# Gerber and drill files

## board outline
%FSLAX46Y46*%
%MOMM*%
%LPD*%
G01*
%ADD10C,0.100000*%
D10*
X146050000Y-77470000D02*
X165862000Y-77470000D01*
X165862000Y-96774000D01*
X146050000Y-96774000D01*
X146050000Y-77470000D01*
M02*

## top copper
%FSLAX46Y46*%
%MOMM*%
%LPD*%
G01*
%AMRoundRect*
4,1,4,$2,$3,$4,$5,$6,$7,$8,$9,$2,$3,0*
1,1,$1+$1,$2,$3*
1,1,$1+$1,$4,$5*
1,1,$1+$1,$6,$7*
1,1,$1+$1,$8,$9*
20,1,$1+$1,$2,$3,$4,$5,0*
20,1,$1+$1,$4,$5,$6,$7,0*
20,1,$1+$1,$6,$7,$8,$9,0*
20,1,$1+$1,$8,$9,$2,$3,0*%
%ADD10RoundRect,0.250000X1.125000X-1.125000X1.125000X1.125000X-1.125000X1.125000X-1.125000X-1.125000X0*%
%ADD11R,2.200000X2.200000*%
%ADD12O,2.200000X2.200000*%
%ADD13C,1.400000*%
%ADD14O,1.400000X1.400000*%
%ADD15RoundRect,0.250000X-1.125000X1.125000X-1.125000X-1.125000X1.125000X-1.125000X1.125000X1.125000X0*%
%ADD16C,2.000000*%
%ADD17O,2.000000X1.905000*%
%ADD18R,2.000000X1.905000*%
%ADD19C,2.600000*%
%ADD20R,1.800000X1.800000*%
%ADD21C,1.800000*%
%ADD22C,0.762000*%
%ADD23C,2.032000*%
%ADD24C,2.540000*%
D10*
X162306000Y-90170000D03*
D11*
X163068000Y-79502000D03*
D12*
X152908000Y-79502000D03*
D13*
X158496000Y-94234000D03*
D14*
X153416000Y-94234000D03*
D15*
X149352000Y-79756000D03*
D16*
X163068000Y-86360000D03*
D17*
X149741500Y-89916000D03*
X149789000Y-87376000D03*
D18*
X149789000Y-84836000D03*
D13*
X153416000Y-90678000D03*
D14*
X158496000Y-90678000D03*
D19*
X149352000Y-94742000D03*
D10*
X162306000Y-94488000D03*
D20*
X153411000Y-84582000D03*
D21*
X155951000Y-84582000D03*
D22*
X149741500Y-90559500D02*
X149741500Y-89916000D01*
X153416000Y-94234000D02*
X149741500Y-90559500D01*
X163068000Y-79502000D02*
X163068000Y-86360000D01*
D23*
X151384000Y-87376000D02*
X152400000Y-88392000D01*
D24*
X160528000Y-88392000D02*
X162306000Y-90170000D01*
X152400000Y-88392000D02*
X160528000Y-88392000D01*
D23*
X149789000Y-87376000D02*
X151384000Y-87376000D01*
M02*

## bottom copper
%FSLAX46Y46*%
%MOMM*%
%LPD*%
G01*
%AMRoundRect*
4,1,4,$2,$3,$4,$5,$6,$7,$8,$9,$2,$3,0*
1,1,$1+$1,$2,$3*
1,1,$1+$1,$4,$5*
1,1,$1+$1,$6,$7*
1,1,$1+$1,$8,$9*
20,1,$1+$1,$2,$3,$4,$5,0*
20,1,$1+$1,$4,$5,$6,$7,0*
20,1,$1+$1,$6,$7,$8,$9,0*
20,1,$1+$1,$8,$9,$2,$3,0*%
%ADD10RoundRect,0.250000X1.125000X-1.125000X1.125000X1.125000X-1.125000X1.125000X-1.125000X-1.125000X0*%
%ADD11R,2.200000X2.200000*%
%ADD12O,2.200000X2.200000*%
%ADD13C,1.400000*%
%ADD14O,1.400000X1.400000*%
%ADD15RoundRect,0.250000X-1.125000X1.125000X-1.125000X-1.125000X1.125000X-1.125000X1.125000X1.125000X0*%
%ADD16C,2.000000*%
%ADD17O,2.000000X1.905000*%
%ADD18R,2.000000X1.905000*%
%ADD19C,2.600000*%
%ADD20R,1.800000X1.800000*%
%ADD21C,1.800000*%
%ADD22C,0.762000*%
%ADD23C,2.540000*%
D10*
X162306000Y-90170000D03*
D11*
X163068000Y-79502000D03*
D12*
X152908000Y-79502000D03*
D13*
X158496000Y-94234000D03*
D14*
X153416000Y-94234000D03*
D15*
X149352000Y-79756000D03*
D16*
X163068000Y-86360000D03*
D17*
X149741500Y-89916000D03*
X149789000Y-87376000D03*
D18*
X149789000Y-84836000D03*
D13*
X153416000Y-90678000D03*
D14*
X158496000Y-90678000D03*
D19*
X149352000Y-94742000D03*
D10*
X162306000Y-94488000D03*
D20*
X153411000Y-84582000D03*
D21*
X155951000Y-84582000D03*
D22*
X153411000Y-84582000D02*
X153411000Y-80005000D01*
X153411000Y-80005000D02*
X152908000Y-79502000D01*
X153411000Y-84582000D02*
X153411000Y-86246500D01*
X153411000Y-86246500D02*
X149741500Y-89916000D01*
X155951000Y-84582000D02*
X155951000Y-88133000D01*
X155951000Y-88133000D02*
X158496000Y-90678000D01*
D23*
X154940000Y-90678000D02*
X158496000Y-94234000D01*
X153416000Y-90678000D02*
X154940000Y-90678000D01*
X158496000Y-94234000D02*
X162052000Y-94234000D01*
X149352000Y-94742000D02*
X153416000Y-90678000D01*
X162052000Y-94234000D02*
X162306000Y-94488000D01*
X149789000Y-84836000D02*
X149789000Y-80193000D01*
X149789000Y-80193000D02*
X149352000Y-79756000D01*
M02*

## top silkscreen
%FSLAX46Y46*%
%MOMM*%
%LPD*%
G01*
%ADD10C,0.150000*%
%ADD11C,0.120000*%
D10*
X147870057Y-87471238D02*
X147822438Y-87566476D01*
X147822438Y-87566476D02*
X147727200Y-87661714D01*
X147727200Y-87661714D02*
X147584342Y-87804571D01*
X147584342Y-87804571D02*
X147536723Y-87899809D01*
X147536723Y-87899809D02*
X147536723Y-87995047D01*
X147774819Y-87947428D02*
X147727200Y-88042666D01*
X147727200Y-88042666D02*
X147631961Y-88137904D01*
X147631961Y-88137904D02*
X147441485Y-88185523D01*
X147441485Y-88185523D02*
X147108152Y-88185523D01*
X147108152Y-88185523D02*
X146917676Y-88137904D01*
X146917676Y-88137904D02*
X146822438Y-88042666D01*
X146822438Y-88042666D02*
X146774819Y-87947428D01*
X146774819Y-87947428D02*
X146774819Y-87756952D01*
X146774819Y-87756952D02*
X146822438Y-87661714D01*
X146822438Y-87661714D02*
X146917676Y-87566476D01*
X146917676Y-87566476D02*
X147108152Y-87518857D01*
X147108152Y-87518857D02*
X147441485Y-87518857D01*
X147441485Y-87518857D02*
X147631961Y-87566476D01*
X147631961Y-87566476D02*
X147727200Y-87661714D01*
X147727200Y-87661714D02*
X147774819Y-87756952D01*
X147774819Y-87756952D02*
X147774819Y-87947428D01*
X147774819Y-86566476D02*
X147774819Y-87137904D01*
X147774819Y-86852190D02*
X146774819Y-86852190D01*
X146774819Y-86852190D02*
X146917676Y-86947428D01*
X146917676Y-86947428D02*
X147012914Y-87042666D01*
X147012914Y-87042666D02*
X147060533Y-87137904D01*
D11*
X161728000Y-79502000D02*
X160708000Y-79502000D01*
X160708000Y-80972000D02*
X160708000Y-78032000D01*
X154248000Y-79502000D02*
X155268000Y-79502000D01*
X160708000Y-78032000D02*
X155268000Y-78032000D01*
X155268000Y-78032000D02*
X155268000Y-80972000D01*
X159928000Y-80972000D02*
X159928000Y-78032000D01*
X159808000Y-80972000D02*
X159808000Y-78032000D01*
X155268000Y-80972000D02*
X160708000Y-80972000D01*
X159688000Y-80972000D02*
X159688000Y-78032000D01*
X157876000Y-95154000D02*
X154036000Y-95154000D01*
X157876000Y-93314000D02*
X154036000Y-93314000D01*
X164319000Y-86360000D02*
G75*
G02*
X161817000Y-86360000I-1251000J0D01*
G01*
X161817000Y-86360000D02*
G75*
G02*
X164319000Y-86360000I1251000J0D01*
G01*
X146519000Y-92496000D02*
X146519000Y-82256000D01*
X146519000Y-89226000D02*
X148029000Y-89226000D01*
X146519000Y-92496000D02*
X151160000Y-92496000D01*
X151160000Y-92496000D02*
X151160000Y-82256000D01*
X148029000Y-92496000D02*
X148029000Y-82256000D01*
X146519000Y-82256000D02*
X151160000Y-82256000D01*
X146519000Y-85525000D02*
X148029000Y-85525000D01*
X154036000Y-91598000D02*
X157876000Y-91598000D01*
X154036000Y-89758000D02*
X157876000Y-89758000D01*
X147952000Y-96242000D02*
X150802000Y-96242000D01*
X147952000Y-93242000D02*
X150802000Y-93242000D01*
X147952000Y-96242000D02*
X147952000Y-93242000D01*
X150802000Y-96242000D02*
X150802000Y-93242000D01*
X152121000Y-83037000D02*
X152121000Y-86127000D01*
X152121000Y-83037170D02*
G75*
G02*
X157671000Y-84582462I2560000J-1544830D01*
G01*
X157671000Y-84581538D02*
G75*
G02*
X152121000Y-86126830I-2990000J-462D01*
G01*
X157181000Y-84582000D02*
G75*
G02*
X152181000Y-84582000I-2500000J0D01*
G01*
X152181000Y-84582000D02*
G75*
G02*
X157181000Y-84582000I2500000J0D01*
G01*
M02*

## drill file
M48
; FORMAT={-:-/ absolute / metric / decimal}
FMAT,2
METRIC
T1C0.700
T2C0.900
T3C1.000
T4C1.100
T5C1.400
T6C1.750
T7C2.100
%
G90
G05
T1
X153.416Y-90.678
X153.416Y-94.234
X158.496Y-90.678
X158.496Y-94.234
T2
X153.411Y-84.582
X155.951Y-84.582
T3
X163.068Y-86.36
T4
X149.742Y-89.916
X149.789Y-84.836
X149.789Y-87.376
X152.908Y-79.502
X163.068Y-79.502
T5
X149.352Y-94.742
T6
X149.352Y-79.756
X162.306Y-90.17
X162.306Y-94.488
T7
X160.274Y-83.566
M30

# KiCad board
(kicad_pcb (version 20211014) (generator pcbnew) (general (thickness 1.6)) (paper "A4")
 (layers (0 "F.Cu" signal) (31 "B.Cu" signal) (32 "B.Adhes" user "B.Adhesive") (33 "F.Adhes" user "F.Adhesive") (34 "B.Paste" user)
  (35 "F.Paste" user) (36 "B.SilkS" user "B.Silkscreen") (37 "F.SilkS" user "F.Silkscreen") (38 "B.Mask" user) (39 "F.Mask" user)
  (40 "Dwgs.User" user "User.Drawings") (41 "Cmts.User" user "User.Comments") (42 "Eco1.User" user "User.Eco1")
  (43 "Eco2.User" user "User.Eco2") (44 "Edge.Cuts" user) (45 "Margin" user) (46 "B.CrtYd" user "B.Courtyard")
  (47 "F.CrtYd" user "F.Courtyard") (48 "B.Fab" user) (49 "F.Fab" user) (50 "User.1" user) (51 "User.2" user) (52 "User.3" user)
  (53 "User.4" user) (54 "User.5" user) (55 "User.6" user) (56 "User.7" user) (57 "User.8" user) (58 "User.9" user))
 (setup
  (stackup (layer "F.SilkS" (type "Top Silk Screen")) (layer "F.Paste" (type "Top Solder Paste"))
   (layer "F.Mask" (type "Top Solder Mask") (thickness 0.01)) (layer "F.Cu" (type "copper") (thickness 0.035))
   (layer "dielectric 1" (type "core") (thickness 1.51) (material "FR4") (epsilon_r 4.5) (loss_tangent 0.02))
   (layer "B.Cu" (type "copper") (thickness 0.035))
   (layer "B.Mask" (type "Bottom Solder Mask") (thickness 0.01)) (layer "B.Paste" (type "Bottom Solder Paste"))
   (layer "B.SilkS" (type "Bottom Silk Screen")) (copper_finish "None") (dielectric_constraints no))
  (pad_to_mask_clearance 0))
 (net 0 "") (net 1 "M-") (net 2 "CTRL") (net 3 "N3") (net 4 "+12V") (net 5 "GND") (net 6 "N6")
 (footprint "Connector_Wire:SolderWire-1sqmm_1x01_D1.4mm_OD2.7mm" (layer "F.Cu") (at 162.306 90.17 90)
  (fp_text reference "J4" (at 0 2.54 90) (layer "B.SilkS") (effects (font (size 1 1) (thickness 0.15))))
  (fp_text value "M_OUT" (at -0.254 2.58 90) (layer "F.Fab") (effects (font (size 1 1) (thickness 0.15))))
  (pad "1" thru_hole roundrect (at 0 0 90) (size 2.75 2.75) (drill 1.75) (layers *.Cu *.Mask) (roundrect_rratio 0.090909) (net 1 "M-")))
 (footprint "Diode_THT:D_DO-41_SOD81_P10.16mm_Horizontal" (layer "F.Cu") (at 163.068 79.502 180)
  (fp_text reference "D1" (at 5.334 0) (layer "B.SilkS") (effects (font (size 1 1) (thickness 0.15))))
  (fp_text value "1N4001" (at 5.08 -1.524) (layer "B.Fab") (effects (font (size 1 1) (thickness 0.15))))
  (fp_line (start 1.34 0) (end 2.36 0) (layer "F.SilkS") (width 0.12))
  (fp_line (start 2.36 -1.47) (end 2.36 1.47) (layer "F.SilkS") (width 0.12))
  (fp_line (start 8.82 0) (end 7.8 0) (layer "F.SilkS") (width 0.12))
  (fp_line (start 2.36 1.47) (end 7.8 1.47) (layer "F.SilkS") (width 0.12))
  (fp_line (start 7.8 1.47) (end 7.8 -1.47) (layer "F.SilkS") (width 0.12))
  (fp_line (start 3.14 -1.47) (end 3.14 1.47) (layer "F.SilkS") (width 0.12))
  (fp_line (start 3.26 -1.47) (end 3.26 1.47) (layer "F.SilkS") (width 0.12))
  (fp_line (start 7.8 -1.47) (end 2.36 -1.47) (layer "F.SilkS") (width 0.12))
  (fp_line (start 3.38 -1.47) (end 3.38 1.47) (layer "F.SilkS") (width 0.12))
  (pad "1" thru_hole rect (at 0 0 180) (size 2.2 2.2) (drill 1.1) (layers *.Cu *.Mask) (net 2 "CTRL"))
  (pad "2" thru_hole oval (at 10.16 0 180) (size 2.2 2.2) (drill 1.1) (layers *.Cu *.Mask) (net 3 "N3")))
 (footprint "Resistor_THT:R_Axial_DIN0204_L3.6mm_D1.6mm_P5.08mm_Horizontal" (layer "F.Cu") (at 158.496 94.234 180)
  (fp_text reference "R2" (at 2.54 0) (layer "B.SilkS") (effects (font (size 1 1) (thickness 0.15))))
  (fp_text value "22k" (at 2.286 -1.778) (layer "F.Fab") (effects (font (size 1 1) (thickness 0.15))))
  (fp_line (start 0.62 -0.92) (end 4.46 -0.92) (layer "F.SilkS") (width 0.12))
  (fp_line (start 0.62 0.92) (end 4.46 0.92) (layer "F.SilkS") (width 0.12))
  (pad "1" thru_hole circle (at 0 0 180) (size 1.4 1.4) (drill 0.7) (layers *.Cu *.Mask) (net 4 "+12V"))
  (pad "2" thru_hole oval (at 5.08 0 180) (size 1.4 1.4) (drill 0.7) (layers *.Cu *.Mask) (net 3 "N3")))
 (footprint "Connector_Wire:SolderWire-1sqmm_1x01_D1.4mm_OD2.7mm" (layer "F.Cu") (at 149.352 79.756 -90)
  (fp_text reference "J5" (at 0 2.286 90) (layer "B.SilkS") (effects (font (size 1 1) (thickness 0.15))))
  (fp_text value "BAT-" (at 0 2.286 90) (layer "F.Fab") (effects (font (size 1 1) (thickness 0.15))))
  (pad "1" thru_hole roundrect (at 0 0 270) (size 2.75 2.75) (drill 1.75) (layers *.Cu *.Mask) (roundrect_rratio 0.090909) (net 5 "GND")))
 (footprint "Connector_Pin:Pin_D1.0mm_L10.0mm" (layer "F.Cu") (at 163.068 86.36 -90)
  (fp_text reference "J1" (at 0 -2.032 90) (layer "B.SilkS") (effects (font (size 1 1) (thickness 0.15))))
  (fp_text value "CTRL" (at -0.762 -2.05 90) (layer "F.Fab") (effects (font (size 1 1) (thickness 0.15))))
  (fp_circle (center 0 0) (end 1.25 0.05) (layer "F.SilkS") (width 0.12) (fill none))
  (pad "1" thru_hole circle (at 0 0 270) (size 2 2) (drill 1) (layers *.Cu *.Mask) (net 2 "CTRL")))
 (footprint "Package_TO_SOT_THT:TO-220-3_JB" (layer "F.Cu") (at 149.789 89.916 90)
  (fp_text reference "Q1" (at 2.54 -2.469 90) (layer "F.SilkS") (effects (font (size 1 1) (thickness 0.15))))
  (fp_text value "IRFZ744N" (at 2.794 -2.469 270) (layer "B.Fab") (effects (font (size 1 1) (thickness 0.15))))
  (fp_line (start -2.58 -3.27) (end 7.66 -3.27) (layer "F.SilkS") (width 0.12))
  (fp_line (start 0.69 -3.27) (end 0.69 -1.76) (layer "F.SilkS") (width 0.12))
  (fp_line (start -2.58 -3.27) (end -2.58 1.371) (layer "F.SilkS") (width 0.12))
  (fp_line (start -2.58 1.371) (end 7.66 1.371) (layer "F.SilkS") (width 0.12))
  (fp_line (start -2.58 -1.76) (end 7.66 -1.76) (layer "F.SilkS") (width 0.12))
  (fp_line (start 7.66 -3.27) (end 7.66 1.371) (layer "F.SilkS") (width 0.12))
  (fp_line (start 4.391 -3.27) (end 4.391 -1.76) (layer "F.SilkS") (width 0.12))
  (pad "1" thru_hole oval (at 0 -0.0475 90) (size 1.905 2) (drill 1.1) (layers *.Cu *.Mask) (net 3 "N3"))
  (pad "2" thru_hole oval (at 2.54 0 90) (size 1.905 2) (drill 1.1) (layers *.Cu *.Mask) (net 1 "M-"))
  (pad "3" thru_hole rect (at 5.08 0 90) (size 1.905 2) (drill 1.1) (layers *.Cu *.Mask) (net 5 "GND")))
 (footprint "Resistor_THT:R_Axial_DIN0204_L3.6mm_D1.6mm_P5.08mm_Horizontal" (layer "F.Cu") (at 153.416 90.678)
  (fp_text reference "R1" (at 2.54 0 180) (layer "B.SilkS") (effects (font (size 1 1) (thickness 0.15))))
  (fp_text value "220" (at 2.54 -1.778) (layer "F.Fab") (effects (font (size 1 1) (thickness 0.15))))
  (fp_line (start 0.62 0.92) (end 4.46 0.92) (layer "F.SilkS") (width 0.12))
  (fp_line (start 0.62 -0.92) (end 4.46 -0.92) (layer "F.SilkS") (width 0.12))
  (pad "1" thru_hole circle (at 0 0) (size 1.4 1.4) (drill 0.7) (layers *.Cu *.Mask) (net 4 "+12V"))
  (pad "2" thru_hole oval (at 5.08 0) (size 1.4 1.4) (drill 0.7) (layers *.Cu *.Mask) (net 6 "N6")))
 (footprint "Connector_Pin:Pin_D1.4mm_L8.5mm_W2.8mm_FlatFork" (layer "F.Cu") (at 149.352 94.742 90)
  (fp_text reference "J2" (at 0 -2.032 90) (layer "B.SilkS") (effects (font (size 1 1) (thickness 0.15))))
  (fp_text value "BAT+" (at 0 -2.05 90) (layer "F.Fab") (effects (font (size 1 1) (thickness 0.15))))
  (fp_line (start -1.5 -1.4) (end -1.5 1.45) (layer "F.SilkS") (width 0.12))
  (fp_line (start 1.5 -1.4) (end 1.5 1.45) (layer "F.SilkS") (width 0.12))
  (fp_line (start -1.5 -1.4) (end 1.5 -1.4) (layer "F.SilkS") (width 0.12))
  (fp_line (start -1.5 1.45) (end 1.5 1.45) (layer "F.SilkS") (width 0.12))
  (pad "1" thru_hole circle (at 0 0 90) (size 2.6 2.6) (drill 1.4) (layers *.Cu *.Mask) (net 4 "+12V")))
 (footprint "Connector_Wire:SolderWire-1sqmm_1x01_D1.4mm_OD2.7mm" (layer "F.Cu") (at 162.306 94.488 90)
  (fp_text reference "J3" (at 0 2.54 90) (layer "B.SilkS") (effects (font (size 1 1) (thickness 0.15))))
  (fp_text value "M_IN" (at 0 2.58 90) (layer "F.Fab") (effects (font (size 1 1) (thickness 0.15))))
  (pad "1" thru_hole roundrect (at 0 0 90) (size 2.75 2.75) (drill 1.75) (layers *.Cu *.Mask) (roundrect_rratio 0.090909) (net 4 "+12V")))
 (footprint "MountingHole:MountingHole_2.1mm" (layer "F.Cu") (at 160.274 83.566 90)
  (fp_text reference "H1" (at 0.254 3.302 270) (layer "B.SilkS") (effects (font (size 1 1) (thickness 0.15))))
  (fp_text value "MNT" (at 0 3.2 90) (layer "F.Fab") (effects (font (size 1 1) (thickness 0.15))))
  (pad "" np_thru_hole circle (at 0 0 90) (size 2.1 2.1) (drill 2.1) (layers *.Cu *.Mask)))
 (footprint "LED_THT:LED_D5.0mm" (layer "F.Cu") (at 153.411 84.582)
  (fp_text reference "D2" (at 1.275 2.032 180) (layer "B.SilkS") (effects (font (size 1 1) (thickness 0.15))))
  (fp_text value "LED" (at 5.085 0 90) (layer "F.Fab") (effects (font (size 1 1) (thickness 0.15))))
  (fp_line (start -1.29 -1.545) (end -1.29 1.545) (layer "F.SilkS") (width 0.12))
  (fp_arc (start -1.29 -1.54483) (mid 2.072002 -2.880433) (end 4.26 0.000462) (layer "F.SilkS") (width 0.12))
  (fp_arc (start 4.26 -0.000462) (mid 2.072002 2.880433) (end -1.29 1.54483) (layer "F.SilkS") (width 0.12))
  (fp_circle (center 1.27 0) (end 3.77 0) (layer "F.SilkS") (width 0.12) (fill none))
  (pad "1" thru_hole rect (at 0 0) (size 1.8 1.8) (drill 0.9) (layers *.Cu *.Mask) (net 3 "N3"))
  (pad "2" thru_hole circle (at 2.54 0) (size 1.8 1.8) (drill 0.9) (layers *.Cu *.Mask) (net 6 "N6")))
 (gr_rect (start 146.05 77.47) (end 165.862 96.774) (layer "Edge.Cuts") (width 0.1) (fill none))
 (segment (start 149.7415 90.5595) (end 149.7415 89.916) (width 0.762) (layer "F.Cu") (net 3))
 (segment (start 153.416 94.234) (end 149.7415 90.5595) (width 0.762) (layer "F.Cu") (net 3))
 (segment (start 153.411 84.582) (end 153.411 80.005) (width 0.762) (layer "B.Cu") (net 3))
 (segment (start 153.411 80.005) (end 152.908 79.502) (width 0.762) (layer "B.Cu") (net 3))
 (segment (start 153.411 84.582) (end 153.411 86.2465) (width 0.762) (layer "B.Cu") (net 3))
 (segment (start 153.411 86.2465) (end 149.7415 89.916) (width 0.762) (layer "B.Cu") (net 3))
 (segment (start 155.951 84.582) (end 155.951 88.133) (width 0.762) (layer "B.Cu") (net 6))
 (segment (start 155.951 88.133) (end 158.496 90.678) (width 0.762) (layer "B.Cu") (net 6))
 (segment (start 154.94 90.678) (end 158.496 94.234) (width 2.54) (layer "B.Cu") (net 4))
 (segment (start 153.416 90.678) (end 154.94 90.678) (width 2.54) (layer "B.Cu") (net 4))
 (segment (start 158.496 94.234) (end 162.052 94.234) (width 2.54) (layer "B.Cu") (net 4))
 (segment (start 149.352 94.742) (end 153.416 90.678) (width 2.54) (layer "B.Cu") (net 4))
 (segment (start 162.052 94.234) (end 162.306 94.488) (width 2.54) (layer "B.Cu") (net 4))
 (segment (start 149.789 84.836) (end 149.789 80.193) (width 2.54) (layer "B.Cu") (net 5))
 (segment (start 149.789 80.193) (end 149.352 79.756) (width 2.54) (layer "B.Cu") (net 5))
 (segment (start 163.068 79.502) (end 163.068 86.36) (width 0.762) (layer "F.Cu") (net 2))
 (segment (start 151.384 87.376) (end 152.4 88.392) (width 2.032) (layer "F.Cu") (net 1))
 (segment (start 160.528 88.392) (end 162.306 90.17) (width 2.54) (layer "F.Cu") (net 1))
 (segment (start 152.4 88.392) (end 160.528 88.392) (width 2.54) (layer "F.Cu") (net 1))
 (segment (start 149.789 87.376) (end 151.384 87.376) (width 2.032) (layer "F.Cu") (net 1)))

